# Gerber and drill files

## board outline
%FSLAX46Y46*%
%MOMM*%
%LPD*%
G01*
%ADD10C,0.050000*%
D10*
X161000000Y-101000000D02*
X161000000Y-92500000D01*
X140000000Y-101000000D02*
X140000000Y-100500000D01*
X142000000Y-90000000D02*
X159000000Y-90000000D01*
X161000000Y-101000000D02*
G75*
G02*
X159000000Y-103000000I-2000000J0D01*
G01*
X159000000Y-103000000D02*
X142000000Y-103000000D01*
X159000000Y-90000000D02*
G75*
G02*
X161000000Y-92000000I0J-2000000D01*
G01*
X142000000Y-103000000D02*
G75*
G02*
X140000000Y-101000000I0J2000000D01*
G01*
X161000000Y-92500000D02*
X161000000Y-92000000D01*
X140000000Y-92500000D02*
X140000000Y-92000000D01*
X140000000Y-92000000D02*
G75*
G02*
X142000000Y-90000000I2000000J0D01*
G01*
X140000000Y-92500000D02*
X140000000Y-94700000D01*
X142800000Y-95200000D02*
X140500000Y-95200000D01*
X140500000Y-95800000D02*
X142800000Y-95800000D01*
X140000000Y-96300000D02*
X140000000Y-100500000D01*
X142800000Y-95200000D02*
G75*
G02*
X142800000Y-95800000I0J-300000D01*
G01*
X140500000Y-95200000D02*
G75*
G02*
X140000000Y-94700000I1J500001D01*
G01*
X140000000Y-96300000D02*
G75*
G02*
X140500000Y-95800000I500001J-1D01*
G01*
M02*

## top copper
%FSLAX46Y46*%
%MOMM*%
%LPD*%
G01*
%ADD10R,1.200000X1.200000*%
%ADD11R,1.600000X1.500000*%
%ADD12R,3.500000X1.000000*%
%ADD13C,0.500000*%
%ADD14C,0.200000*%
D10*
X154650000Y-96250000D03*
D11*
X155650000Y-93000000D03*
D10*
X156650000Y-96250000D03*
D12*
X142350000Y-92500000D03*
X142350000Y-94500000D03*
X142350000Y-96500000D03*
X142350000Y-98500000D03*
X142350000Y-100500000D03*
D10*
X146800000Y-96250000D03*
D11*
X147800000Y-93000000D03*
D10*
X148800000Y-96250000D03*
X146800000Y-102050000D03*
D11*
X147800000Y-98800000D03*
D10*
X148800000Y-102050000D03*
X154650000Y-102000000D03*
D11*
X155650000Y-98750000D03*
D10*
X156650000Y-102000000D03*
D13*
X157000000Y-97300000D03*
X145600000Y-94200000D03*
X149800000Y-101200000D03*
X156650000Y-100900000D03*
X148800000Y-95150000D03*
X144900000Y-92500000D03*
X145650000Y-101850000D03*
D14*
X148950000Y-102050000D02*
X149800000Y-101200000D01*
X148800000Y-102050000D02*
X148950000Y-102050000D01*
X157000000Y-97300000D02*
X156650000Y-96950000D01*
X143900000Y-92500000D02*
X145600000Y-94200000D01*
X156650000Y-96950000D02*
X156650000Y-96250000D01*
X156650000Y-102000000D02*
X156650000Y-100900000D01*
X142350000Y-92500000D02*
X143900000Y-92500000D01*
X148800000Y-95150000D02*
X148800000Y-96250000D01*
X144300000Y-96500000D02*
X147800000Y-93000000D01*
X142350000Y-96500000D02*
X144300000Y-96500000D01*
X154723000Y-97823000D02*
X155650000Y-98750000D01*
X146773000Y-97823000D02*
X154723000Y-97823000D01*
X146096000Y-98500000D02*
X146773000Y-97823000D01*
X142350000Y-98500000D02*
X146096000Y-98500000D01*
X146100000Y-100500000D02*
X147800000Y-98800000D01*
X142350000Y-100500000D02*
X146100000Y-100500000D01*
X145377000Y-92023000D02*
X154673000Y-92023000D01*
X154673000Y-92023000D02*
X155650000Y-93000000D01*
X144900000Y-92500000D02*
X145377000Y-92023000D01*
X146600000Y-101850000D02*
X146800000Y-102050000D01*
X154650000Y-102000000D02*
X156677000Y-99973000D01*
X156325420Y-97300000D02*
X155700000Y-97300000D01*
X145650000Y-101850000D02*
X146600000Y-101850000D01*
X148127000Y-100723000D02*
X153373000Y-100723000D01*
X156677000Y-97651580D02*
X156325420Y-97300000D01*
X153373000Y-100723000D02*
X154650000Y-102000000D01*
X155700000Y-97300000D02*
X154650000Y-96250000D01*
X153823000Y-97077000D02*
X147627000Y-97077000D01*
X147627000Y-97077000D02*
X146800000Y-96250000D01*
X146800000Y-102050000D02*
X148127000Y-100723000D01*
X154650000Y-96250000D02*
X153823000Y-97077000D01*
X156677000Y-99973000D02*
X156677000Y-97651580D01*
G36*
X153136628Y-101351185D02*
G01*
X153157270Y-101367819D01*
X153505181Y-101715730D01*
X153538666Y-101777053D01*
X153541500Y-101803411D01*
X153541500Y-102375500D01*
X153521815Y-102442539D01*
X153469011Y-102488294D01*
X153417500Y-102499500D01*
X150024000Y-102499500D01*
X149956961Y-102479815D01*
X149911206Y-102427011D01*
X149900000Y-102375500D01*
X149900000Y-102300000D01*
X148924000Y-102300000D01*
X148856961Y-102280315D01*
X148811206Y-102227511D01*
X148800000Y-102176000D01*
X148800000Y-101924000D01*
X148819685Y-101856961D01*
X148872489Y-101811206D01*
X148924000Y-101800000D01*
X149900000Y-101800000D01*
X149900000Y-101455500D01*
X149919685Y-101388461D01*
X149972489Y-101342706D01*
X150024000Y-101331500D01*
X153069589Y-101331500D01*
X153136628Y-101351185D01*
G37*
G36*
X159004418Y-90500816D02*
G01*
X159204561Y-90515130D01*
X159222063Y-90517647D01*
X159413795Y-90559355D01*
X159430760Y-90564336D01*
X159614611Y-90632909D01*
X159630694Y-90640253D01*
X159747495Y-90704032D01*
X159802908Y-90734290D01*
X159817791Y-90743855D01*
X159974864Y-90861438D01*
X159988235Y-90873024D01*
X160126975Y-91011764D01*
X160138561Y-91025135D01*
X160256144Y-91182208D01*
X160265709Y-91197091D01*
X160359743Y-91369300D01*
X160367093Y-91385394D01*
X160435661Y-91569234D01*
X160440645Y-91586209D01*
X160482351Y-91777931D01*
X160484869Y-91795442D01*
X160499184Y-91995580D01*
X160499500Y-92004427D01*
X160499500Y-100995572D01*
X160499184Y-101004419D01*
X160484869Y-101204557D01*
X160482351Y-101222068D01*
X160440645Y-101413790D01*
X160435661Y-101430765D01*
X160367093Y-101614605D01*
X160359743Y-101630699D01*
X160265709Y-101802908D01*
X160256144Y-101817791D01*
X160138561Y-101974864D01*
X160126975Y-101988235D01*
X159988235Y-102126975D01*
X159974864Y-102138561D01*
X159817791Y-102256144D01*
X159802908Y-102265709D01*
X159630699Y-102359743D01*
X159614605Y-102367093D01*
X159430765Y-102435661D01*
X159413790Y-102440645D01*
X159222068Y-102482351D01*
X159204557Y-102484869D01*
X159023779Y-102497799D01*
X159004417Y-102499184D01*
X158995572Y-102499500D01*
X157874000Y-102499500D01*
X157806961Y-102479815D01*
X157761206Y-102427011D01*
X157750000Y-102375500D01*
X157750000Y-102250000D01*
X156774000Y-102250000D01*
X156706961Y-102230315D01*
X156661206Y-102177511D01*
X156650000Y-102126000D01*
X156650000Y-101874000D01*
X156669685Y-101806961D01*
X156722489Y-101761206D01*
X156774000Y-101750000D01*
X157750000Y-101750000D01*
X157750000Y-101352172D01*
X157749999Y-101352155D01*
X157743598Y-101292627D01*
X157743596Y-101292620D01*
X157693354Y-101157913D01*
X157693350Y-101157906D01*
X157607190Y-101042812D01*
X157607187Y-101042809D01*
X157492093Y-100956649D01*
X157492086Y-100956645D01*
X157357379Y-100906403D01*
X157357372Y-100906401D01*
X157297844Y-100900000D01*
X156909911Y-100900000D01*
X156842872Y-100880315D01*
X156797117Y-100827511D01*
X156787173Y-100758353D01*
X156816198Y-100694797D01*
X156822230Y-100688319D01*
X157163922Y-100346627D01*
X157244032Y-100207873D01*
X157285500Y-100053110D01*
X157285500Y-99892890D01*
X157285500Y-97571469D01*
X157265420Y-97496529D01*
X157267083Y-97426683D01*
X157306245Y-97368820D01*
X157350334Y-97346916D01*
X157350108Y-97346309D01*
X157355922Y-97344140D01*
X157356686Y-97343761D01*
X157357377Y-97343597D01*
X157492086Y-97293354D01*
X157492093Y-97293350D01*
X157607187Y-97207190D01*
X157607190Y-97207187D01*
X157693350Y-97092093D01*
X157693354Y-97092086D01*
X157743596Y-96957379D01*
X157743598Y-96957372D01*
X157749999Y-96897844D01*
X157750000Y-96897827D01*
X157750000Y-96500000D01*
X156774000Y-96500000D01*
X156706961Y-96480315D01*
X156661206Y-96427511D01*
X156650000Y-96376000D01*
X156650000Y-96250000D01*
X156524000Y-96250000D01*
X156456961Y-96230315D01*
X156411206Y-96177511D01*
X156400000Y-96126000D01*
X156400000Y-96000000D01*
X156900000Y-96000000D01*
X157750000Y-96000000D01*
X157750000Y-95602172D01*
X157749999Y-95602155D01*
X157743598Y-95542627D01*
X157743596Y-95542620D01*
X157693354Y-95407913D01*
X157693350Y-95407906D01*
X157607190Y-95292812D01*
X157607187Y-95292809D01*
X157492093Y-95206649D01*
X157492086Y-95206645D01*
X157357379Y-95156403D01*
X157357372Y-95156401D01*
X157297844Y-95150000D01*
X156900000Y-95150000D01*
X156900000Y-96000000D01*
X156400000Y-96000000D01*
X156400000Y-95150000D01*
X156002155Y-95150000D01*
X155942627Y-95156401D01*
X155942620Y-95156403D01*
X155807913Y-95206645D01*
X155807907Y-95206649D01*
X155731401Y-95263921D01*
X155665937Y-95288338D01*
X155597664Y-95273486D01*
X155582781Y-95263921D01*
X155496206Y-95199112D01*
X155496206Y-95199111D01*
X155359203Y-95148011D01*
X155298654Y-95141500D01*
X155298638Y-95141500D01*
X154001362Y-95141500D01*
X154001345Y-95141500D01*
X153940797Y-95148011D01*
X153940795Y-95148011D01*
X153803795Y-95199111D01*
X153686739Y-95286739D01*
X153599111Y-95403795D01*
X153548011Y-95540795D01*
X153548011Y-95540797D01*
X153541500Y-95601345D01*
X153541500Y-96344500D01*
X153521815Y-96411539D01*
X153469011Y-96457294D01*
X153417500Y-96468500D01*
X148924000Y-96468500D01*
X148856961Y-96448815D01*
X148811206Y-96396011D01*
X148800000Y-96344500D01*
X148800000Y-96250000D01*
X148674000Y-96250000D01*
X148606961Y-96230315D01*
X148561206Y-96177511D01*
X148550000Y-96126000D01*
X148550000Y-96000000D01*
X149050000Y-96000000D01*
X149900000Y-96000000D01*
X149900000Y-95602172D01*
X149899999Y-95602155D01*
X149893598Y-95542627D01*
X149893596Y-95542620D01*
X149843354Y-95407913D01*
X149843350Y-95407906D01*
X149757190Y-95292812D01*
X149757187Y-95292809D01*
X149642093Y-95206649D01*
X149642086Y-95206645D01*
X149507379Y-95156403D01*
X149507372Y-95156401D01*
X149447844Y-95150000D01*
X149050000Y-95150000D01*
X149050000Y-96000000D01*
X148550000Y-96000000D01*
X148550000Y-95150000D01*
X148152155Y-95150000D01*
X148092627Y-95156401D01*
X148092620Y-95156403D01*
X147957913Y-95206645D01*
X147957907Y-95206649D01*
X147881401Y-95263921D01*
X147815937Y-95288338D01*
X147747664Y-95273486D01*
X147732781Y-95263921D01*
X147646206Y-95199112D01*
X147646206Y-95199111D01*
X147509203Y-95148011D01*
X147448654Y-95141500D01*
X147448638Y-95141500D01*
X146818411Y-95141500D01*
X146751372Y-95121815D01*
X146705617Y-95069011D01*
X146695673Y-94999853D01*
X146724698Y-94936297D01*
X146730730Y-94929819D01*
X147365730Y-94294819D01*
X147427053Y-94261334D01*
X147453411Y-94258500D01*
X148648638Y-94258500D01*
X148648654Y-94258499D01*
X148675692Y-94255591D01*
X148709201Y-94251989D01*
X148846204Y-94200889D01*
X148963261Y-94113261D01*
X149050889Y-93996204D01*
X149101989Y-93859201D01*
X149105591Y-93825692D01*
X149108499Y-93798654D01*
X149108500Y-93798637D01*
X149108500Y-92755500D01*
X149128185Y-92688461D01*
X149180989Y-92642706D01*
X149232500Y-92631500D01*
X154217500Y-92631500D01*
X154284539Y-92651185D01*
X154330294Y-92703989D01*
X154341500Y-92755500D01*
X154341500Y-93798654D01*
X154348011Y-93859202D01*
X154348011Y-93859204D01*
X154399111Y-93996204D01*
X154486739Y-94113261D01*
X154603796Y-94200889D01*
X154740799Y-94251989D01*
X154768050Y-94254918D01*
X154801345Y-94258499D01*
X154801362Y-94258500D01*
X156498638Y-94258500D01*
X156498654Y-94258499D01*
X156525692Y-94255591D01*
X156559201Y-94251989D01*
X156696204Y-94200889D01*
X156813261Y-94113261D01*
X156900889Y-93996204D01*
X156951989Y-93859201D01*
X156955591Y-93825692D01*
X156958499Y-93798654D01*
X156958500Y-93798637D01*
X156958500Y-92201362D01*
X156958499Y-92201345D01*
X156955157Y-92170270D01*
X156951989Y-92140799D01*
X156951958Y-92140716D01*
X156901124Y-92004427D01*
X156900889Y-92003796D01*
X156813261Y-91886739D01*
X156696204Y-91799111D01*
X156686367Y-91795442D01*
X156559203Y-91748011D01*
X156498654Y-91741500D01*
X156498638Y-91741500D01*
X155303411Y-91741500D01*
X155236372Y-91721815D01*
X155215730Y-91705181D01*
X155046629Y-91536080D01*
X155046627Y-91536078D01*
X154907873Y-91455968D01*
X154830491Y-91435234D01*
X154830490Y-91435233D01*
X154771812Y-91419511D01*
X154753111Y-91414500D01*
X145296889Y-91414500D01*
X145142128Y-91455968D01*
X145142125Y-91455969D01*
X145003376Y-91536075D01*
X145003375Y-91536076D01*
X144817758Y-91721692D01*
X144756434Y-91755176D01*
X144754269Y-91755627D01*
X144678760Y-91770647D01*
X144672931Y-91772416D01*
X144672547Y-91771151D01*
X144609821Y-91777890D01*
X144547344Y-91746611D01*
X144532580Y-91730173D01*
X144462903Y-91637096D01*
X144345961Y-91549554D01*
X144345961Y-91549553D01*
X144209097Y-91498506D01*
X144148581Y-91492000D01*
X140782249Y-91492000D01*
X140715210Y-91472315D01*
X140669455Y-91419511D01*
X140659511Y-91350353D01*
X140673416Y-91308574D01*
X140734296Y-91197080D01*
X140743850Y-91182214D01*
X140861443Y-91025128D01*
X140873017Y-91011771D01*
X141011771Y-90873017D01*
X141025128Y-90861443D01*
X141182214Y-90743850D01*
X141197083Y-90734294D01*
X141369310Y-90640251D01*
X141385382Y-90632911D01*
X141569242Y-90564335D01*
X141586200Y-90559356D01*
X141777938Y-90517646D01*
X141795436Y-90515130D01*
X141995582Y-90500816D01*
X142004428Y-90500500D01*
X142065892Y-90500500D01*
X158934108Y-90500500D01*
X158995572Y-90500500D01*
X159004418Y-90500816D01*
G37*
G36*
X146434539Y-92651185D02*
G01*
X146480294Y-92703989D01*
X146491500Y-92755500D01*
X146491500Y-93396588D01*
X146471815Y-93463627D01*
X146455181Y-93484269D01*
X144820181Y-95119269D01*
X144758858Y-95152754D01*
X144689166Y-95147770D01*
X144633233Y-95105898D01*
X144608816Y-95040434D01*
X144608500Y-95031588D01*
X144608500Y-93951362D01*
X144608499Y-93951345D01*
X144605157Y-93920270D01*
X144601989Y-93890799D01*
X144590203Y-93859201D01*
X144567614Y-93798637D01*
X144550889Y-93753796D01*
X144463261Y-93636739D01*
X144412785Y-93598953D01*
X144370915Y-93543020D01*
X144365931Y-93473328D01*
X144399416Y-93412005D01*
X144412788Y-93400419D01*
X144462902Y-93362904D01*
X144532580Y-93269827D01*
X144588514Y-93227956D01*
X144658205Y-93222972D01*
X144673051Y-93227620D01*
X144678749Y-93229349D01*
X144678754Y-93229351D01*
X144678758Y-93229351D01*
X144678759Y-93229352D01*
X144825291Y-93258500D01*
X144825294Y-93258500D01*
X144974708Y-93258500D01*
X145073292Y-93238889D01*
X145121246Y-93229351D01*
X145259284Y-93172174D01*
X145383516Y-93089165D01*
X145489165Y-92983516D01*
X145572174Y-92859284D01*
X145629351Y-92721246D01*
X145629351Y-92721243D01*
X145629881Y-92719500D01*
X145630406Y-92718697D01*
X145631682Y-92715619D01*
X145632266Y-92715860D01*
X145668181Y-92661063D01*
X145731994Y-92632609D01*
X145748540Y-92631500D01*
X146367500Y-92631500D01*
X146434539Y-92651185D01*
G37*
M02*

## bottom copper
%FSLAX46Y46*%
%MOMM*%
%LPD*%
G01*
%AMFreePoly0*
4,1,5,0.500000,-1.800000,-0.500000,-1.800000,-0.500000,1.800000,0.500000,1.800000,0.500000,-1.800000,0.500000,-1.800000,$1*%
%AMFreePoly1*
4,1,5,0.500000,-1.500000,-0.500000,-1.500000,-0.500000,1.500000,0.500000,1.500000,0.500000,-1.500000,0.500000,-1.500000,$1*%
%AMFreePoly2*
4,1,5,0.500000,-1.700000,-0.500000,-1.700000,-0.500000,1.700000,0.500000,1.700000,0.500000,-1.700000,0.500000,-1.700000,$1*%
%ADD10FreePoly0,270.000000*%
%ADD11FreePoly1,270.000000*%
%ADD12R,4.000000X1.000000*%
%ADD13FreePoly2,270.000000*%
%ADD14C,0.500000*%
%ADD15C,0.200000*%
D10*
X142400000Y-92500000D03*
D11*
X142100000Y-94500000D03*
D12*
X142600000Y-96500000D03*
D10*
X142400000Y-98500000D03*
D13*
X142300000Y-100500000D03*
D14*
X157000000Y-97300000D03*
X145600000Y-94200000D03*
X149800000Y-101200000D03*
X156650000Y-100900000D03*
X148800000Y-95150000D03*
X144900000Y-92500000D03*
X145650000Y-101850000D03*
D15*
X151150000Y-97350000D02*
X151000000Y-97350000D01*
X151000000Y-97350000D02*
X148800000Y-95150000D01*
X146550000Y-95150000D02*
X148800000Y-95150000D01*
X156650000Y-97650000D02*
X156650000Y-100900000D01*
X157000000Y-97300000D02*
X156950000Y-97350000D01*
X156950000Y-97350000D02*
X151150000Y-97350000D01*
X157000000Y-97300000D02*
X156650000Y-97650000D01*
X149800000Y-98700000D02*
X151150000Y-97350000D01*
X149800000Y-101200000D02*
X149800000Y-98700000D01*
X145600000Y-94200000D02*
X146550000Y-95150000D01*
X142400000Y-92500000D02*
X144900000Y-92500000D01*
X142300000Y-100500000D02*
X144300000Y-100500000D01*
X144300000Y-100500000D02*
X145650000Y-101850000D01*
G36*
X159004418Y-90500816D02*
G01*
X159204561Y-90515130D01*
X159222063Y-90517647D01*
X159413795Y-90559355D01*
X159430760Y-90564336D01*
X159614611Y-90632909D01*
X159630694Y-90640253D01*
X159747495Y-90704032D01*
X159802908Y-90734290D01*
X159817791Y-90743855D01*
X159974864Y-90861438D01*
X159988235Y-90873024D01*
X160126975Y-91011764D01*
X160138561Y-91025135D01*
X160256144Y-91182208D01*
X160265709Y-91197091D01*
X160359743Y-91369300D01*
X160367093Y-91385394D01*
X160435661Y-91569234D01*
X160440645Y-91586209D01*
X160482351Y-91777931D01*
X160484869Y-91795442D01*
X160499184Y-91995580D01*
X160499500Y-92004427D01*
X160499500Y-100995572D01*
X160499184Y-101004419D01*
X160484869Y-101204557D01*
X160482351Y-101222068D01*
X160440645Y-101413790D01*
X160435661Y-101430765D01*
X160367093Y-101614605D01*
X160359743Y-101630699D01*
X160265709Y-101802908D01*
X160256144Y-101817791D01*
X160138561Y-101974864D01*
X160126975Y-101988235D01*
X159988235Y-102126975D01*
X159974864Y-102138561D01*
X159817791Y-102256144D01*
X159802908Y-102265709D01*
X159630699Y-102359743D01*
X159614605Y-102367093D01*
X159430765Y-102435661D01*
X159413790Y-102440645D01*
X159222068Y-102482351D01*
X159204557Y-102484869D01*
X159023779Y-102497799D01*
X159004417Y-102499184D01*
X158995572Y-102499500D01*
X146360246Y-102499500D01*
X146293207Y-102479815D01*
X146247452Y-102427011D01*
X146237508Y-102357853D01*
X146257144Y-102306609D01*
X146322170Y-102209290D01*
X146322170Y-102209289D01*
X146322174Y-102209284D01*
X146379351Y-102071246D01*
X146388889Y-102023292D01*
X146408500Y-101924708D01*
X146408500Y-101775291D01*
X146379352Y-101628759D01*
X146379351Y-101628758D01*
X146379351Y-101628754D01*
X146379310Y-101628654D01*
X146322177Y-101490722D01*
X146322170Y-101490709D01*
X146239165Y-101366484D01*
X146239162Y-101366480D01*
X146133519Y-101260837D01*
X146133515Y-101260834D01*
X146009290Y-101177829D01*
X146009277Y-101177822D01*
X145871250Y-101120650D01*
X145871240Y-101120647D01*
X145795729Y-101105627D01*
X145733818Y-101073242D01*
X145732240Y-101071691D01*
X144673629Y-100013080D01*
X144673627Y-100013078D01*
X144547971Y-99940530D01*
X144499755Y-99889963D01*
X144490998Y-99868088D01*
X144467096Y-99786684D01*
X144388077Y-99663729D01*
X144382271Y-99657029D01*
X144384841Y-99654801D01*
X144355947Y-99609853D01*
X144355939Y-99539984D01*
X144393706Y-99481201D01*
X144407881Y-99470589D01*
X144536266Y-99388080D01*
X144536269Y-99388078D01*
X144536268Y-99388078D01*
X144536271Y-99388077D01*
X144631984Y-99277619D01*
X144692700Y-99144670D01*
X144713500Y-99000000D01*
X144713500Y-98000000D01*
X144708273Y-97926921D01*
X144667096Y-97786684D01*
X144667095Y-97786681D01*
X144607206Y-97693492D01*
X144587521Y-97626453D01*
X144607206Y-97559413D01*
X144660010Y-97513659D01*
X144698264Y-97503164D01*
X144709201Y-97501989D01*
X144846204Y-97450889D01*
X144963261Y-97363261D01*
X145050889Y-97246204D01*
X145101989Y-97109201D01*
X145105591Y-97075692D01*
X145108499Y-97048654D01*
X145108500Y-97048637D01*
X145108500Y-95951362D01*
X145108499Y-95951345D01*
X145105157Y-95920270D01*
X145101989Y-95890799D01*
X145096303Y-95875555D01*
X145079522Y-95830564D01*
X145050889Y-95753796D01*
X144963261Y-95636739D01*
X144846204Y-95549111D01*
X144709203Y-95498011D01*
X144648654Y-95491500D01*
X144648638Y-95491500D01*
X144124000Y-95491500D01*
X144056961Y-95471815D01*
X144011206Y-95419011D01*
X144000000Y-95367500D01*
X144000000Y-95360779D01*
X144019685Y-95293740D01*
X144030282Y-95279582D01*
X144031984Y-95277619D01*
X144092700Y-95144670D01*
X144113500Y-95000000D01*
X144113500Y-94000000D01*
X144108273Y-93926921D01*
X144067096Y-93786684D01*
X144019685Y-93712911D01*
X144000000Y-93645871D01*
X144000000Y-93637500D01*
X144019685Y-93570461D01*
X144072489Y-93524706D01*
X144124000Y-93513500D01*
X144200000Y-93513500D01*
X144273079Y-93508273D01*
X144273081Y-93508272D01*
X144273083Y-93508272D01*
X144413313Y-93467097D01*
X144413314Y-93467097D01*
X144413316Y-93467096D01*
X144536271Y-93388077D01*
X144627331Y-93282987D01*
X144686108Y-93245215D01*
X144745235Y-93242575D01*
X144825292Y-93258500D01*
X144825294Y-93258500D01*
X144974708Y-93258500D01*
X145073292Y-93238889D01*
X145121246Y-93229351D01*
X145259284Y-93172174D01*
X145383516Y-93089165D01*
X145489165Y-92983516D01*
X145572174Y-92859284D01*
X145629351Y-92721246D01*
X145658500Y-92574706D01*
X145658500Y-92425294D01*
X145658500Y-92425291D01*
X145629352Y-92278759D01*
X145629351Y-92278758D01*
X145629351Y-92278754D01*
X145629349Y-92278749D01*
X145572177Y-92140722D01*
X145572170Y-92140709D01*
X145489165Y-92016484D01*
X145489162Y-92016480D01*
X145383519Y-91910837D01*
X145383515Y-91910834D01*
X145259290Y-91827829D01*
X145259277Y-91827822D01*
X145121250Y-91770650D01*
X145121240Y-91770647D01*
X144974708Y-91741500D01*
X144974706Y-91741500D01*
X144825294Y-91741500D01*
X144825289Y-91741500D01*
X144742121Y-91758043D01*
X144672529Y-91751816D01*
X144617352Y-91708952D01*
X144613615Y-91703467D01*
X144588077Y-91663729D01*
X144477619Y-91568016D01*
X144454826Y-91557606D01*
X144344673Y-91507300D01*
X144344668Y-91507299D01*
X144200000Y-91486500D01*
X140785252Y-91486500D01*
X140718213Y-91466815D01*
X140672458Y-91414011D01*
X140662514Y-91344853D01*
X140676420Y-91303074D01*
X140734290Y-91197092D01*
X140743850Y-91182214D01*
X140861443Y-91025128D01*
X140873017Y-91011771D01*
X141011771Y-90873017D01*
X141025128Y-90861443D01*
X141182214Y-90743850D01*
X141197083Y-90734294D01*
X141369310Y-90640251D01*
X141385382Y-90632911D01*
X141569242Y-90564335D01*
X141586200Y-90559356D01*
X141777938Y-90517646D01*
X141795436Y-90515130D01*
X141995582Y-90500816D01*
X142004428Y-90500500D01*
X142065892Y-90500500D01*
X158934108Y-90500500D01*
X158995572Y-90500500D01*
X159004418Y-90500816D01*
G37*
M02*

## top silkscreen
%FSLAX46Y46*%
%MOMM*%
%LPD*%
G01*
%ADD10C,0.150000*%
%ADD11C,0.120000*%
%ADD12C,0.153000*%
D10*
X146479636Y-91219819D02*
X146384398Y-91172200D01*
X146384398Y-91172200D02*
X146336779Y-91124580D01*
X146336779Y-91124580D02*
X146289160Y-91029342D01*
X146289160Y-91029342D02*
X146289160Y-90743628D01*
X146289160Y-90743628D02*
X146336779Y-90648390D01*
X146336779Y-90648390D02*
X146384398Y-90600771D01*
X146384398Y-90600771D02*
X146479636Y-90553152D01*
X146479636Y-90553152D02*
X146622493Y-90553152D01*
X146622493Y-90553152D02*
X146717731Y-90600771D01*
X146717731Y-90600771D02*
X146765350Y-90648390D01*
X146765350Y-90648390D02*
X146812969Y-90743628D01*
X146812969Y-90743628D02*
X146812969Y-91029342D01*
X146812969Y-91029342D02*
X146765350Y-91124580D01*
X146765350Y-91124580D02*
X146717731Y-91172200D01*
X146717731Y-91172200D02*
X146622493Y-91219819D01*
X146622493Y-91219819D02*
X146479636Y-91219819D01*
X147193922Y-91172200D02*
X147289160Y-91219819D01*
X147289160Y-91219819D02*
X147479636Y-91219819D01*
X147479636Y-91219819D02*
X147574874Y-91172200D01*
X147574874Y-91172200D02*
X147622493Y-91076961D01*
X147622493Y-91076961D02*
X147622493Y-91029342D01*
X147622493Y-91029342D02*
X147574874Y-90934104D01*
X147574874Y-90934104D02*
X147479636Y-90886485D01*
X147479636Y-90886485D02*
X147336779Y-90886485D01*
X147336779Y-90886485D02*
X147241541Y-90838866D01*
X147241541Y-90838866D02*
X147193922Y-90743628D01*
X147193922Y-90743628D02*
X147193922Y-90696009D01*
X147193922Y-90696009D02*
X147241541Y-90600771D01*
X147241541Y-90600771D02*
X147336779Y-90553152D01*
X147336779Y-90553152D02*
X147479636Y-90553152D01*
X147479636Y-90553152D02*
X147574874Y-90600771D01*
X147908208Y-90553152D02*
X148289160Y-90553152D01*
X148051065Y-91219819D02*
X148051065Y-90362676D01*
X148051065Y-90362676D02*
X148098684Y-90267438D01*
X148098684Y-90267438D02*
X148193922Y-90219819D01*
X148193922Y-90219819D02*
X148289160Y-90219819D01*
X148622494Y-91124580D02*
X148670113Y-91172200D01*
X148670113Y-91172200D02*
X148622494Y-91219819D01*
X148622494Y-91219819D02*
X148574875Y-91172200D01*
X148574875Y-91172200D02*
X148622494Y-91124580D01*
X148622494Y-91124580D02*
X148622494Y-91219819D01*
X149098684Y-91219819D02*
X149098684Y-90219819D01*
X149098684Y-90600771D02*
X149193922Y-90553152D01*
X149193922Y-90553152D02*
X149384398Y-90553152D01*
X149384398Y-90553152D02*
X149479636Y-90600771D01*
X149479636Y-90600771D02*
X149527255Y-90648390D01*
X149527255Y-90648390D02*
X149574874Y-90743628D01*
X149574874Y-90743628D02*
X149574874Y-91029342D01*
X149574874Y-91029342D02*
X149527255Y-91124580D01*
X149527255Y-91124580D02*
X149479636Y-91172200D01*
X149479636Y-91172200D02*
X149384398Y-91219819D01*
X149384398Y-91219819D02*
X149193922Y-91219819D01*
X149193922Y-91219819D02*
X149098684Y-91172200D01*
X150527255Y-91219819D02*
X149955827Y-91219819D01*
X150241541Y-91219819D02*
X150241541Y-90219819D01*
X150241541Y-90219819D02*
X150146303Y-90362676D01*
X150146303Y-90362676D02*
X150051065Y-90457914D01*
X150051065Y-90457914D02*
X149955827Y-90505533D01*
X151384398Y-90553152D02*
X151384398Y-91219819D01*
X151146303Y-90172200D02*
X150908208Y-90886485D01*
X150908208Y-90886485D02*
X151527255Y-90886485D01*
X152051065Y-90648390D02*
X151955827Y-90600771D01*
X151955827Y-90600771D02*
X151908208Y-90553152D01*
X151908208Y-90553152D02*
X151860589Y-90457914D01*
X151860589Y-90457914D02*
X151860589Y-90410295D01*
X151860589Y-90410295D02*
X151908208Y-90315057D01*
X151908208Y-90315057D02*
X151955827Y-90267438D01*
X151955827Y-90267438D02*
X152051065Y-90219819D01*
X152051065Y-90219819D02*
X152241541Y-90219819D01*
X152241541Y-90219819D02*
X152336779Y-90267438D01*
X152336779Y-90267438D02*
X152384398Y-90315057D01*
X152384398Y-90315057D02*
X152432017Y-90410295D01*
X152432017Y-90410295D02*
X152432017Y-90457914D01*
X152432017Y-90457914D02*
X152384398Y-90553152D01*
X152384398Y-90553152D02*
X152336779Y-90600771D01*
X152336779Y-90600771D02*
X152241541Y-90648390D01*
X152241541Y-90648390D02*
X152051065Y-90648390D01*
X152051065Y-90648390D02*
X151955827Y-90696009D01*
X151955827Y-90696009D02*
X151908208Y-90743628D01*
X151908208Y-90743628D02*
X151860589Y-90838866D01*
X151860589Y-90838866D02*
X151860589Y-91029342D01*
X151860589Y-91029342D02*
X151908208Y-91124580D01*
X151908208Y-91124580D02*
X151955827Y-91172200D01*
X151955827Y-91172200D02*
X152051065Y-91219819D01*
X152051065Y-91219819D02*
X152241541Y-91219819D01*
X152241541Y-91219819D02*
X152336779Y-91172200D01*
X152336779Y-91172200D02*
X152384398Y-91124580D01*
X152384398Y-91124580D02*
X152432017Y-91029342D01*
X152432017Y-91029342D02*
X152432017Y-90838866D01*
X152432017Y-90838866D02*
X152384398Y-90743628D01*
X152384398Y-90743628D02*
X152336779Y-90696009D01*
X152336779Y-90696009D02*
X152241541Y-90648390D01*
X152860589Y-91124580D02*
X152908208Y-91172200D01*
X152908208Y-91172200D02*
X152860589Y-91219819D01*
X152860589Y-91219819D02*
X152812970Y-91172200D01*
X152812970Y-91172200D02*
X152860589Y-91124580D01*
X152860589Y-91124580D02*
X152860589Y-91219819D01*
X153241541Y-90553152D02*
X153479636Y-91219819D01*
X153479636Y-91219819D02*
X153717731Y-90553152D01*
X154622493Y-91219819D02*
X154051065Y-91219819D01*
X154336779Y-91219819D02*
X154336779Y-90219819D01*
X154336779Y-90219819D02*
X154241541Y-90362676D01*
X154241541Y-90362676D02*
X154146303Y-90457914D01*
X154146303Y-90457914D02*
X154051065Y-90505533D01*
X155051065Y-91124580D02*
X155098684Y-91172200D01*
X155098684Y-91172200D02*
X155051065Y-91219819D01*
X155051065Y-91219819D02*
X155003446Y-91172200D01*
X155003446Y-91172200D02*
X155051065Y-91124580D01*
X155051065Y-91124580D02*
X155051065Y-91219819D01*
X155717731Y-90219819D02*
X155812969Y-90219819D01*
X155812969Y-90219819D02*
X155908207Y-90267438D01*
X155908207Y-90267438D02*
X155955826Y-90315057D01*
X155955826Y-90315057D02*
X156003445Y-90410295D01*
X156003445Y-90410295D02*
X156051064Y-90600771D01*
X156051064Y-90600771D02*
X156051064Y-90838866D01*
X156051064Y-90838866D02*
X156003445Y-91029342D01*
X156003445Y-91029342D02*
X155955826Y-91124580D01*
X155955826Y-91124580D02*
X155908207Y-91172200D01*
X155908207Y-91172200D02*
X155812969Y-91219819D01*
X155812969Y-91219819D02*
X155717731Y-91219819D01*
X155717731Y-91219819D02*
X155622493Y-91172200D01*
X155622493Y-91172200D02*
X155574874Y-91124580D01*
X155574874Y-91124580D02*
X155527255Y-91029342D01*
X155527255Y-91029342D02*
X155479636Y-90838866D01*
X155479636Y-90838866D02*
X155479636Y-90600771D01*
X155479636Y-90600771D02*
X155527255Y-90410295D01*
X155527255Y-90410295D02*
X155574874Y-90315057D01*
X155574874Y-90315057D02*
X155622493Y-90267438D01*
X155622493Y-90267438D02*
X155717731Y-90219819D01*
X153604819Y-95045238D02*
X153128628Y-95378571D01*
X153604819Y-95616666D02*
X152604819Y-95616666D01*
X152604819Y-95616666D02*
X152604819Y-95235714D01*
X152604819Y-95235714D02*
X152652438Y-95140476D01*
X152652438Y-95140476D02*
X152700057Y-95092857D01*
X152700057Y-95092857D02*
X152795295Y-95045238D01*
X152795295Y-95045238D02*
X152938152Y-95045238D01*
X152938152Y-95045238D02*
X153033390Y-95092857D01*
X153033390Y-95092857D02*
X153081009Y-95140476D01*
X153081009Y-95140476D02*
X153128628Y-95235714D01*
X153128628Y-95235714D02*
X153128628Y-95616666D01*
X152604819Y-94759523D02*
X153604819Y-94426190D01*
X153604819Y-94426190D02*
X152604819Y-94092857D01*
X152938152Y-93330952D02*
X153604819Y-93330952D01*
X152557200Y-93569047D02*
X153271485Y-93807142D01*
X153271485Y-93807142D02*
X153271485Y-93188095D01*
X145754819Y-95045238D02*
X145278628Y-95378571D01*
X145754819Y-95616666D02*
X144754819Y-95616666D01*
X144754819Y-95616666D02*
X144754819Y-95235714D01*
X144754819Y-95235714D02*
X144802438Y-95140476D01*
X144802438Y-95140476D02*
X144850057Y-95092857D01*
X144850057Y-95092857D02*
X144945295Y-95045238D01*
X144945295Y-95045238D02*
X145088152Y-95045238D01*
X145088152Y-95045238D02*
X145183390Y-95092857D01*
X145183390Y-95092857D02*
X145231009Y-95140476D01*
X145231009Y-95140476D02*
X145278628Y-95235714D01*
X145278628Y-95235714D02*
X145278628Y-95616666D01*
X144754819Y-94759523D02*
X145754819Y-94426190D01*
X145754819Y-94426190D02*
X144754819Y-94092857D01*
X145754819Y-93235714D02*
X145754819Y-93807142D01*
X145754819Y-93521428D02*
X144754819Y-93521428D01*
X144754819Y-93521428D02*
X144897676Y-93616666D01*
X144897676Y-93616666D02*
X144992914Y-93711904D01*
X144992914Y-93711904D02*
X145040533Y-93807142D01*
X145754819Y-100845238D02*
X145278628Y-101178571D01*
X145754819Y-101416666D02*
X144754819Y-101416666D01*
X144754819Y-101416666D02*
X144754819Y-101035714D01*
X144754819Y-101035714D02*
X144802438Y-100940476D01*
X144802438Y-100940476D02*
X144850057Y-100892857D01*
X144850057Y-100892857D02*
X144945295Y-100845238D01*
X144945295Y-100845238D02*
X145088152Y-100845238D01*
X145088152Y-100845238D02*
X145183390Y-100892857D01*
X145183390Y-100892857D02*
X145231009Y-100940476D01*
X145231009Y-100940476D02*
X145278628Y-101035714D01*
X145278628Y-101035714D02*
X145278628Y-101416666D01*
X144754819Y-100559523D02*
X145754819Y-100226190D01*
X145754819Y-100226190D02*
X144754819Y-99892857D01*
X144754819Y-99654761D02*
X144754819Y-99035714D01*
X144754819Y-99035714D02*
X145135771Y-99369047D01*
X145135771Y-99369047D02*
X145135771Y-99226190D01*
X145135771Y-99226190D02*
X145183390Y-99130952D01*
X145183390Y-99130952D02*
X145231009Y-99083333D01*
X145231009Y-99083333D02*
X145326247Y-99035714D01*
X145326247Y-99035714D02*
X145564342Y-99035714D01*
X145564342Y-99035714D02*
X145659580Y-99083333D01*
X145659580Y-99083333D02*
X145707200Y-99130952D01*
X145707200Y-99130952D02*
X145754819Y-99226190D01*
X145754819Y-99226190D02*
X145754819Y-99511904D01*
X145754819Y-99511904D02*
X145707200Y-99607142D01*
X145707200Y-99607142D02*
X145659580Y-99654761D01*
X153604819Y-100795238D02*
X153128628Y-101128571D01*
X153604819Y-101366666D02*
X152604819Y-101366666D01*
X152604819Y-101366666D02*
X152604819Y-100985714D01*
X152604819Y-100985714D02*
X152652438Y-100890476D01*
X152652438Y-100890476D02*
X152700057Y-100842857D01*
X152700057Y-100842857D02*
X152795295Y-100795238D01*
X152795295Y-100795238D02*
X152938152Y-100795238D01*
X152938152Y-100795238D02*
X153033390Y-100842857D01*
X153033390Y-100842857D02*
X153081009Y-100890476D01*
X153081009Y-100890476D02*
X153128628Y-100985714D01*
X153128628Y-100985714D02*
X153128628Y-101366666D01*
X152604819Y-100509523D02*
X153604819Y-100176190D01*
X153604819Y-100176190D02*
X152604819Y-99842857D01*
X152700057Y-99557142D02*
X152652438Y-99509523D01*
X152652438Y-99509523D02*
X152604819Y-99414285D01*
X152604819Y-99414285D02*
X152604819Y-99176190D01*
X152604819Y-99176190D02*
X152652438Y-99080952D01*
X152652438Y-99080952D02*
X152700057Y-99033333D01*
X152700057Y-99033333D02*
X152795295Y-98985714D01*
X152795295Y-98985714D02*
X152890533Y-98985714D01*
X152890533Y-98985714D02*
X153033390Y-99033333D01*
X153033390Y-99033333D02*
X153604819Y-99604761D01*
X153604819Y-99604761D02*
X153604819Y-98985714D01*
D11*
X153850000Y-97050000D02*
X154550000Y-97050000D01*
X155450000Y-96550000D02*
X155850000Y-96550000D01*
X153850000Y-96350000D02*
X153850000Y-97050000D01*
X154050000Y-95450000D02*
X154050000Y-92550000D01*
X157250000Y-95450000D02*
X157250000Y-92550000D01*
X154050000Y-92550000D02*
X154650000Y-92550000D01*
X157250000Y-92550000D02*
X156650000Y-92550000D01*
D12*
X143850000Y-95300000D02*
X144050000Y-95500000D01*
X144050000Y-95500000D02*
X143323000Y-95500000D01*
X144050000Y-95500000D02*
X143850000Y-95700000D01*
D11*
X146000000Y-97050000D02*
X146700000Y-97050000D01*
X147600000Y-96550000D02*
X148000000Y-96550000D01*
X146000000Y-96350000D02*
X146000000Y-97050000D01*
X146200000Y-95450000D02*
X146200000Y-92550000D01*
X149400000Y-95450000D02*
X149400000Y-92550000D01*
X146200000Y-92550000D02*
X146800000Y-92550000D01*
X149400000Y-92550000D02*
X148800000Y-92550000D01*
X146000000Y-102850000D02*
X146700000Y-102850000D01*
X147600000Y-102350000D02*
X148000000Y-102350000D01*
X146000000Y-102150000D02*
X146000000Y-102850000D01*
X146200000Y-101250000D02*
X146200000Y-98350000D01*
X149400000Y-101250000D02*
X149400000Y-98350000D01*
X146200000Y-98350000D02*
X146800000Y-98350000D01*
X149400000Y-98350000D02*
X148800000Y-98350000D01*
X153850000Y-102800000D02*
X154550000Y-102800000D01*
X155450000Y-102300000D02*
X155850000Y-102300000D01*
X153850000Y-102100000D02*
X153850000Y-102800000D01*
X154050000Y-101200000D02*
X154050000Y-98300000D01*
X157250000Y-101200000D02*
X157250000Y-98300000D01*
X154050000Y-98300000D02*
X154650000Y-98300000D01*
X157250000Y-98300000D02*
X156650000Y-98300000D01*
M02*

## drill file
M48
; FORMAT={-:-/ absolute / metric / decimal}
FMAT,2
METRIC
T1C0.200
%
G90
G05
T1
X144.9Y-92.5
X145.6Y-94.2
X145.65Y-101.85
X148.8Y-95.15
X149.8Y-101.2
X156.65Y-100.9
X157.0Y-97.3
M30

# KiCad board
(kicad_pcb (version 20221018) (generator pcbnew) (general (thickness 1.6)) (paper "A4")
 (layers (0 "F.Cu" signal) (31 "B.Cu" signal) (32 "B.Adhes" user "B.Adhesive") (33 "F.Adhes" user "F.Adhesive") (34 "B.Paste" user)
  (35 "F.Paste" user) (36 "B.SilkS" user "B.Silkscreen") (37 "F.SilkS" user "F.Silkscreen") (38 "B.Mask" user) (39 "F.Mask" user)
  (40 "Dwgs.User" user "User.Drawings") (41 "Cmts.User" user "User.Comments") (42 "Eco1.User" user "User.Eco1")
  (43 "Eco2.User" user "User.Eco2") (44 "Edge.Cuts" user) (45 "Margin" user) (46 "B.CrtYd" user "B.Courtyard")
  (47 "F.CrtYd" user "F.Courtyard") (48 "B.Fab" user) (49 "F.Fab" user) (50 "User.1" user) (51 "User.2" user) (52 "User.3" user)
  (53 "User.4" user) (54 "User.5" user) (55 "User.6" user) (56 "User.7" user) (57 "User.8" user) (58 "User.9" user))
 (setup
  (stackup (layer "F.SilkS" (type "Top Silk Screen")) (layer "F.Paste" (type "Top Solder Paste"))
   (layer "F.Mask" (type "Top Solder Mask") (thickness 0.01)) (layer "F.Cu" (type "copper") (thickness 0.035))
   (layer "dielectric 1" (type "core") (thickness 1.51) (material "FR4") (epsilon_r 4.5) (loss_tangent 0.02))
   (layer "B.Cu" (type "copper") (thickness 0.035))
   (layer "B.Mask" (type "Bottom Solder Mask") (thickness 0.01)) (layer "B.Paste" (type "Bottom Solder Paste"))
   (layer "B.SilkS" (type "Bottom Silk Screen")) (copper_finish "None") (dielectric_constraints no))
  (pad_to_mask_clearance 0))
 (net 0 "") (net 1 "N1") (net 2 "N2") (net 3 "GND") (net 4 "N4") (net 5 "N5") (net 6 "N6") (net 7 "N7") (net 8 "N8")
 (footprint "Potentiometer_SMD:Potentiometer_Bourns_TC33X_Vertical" (layer "F.Cu") (at 155.65 94.45 90)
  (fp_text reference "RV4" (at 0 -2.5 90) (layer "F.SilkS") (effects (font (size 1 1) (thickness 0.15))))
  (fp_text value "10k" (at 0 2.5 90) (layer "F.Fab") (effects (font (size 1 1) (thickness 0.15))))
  (fp_line (start -2.6 -1.8) (end -2.6 -1.1) (stroke (width 0.12) (type solid)) (layer "F.SilkS"))
  (fp_line (start -2.1 -0.2) (end -2.1 0.2) (stroke (width 0.12) (type solid)) (layer "F.SilkS"))
  (fp_line (start -1.9 -1.8) (end -2.6 -1.8) (stroke (width 0.12) (type solid)) (layer "F.SilkS"))
  (fp_line (start -1 -1.6) (end 1.9 -1.6) (stroke (width 0.12) (type solid)) (layer "F.SilkS"))
  (fp_line (start -1 1.6) (end 1.9 1.6) (stroke (width 0.12) (type solid)) (layer "F.SilkS"))
  (fp_line (start 1.9 -1.6) (end 1.9 -1) (stroke (width 0.12) (type solid)) (layer "F.SilkS"))
  (fp_line (start 1.9 1.6) (end 1.9 1) (stroke (width 0.12) (type solid)) (layer "F.SilkS"))
  (pad "1" smd rect (at -1.8 -1 90) (size 1.2 1.2) (layers "F.Cu" "F.Paste" "F.Mask") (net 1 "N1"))
  (pad "2" smd rect (at 1.45 0 90) (size 1.5 1.6) (layers "F.Cu" "F.Paste" "F.Mask") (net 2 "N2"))
  (pad "3" smd rect (at -1.8 1 90) (size 1.2 1.2) (layers "F.Cu" "F.Paste" "F.Mask") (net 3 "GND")))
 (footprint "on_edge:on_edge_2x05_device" (layer "F.Cu") (at 140 96.5 -90)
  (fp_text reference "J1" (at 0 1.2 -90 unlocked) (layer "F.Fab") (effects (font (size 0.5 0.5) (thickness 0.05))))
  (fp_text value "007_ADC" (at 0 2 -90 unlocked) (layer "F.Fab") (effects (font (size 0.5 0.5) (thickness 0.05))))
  (fp_line (start -1.2 -3.85) (end -1 -4.05) (stroke (width 0.153) (type solid)) (layer "F.SilkS"))
  (fp_line (start -1 -4.05) (end -1 -3.323) (stroke (width 0.153) (type solid)) (layer "F.SilkS"))
  (fp_line (start -1 -4.05) (end -0.8 -3.85) (stroke (width 0.153) (type solid)) (layer "F.SilkS"))
  (fp_line (start -4 0) (end -1.8 0) (stroke (width 0.05) (type solid)) (layer "Edge.Cuts"))
  (fp_line (start -1.3 -2.8) (end -1.3 -0.5) (stroke (width 0.05) (type solid)) (layer "Edge.Cuts"))
  (fp_line (start -0.7 -0.5) (end -0.7 -2.8) (stroke (width 0.05) (type solid)) (layer "Edge.Cuts"))
  (fp_line (start -0.2 0) (end 4 0) (stroke (width 0.05) (type solid)) (layer "Edge.Cuts"))
  (fp_arc (start -1.3 -2.8) (mid -1 -3.1) (end -0.7 -2.8) (stroke (width 0.05) (type solid)) (layer "Edge.Cuts"))
  (fp_arc (start -1.3 -0.5) (mid -1.446447 -0.146447) (end -1.8 0) (stroke (width 0.05) (type solid)) (layer "Edge.Cuts"))
  (fp_arc (start -0.2 0) (mid -0.553553 -0.146447) (end -0.7 -0.5) (stroke (width 0.05) (type solid)) (layer "Edge.Cuts"))
  (pad "1" smd rect (at -4 -2.35 90) (size 1 3.5) (layers "F.Cu" "F.Mask") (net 3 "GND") (zone_connect 0))
  (pad "2" smd rect (at -2 -2.35 270) (size 1 3.5) (layers "F.Cu" "F.Mask") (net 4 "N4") (zone_connect 0))
  (pad "3" smd rect (at 0 -2.35 270) (size 1 3.5) (layers "F.Cu" "F.Mask") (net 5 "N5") (zone_connect 0))
  (pad "4" smd rect (at 2 -2.35 90) (size 1 3.5) (layers "F.Cu" "F.Mask") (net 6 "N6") (zone_connect 0))
  (pad "5" smd rect (at 4 -2.35 90) (size 1 3.5) (layers "F.Cu" "F.Mask") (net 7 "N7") (zone_connect 0))
  (pad "6" smd custom (at -4 -2.4 270) (size 1 3.6) (layers "B.Cu" "B.Mask") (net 2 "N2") (zone_connect 0)
   (options (clearance outline) (anchor rect)) (primitives))
  (pad "7" smd custom (at -2 -2.1 270) (size 1 3) (layers "B.Cu" "B.Mask") (zone_connect 0) (options (clearance outline) (anchor rect))
   (primitives))
  (pad "8" smd rect (at 0 -2.6 270) (size 1 4) (layers "B.Cu" "B.Mask") (zone_connect 0))
  (pad "9" smd custom (at 2 -2.4 270) (size 1 3.6) (layers "B.Cu" "B.Mask") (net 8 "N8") (zone_connect 0)
   (options (clearance outline) (anchor rect)) (primitives))
  (pad "10" smd custom (at 4 -2.3 270) (size 1 3.4) (layers "B.Cu" "B.Mask") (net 1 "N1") (zone_connect 0)
   (options (clearance outline) (anchor rect)) (primitives))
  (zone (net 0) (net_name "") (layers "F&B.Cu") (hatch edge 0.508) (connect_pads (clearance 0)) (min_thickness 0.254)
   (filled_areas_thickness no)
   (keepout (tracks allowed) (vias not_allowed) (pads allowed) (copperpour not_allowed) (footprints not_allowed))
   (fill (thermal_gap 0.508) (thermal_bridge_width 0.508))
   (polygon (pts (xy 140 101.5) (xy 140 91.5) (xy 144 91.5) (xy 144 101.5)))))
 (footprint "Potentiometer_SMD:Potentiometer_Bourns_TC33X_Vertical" (layer "F.Cu") (at 147.8 94.45 90)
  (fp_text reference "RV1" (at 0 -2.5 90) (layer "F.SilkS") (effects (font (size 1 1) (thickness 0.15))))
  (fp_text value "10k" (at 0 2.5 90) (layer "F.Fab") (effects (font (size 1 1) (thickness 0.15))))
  (fp_line (start -2.6 -1.8) (end -2.6 -1.1) (stroke (width 0.12) (type solid)) (layer "F.SilkS"))
  (fp_line (start -2.1 -0.2) (end -2.1 0.2) (stroke (width 0.12) (type solid)) (layer "F.SilkS"))
  (fp_line (start -1.9 -1.8) (end -2.6 -1.8) (stroke (width 0.12) (type solid)) (layer "F.SilkS"))
  (fp_line (start -1 -1.6) (end 1.9 -1.6) (stroke (width 0.12) (type solid)) (layer "F.SilkS"))
  (fp_line (start -1 1.6) (end 1.9 1.6) (stroke (width 0.12) (type solid)) (layer "F.SilkS"))
  (fp_line (start 1.9 -1.6) (end 1.9 -1) (stroke (width 0.12) (type solid)) (layer "F.SilkS"))
  (fp_line (start 1.9 1.6) (end 1.9 1) (stroke (width 0.12) (type solid)) (layer "F.SilkS"))
  (pad "1" smd rect (at -1.8 -1 90) (size 1.2 1.2) (layers "F.Cu" "F.Paste" "F.Mask") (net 1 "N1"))
  (pad "2" smd rect (at 1.45 0 90) (size 1.5 1.6) (layers "F.Cu" "F.Paste" "F.Mask") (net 5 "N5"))
  (pad "3" smd rect (at -1.8 1 90) (size 1.2 1.2) (layers "F.Cu" "F.Paste" "F.Mask") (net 3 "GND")))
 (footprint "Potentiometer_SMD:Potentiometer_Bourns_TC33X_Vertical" (layer "F.Cu") (at 147.8 100.25 90)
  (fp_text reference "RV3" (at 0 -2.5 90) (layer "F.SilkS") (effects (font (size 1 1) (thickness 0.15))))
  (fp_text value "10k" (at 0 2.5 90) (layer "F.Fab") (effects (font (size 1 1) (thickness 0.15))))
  (fp_line (start -2.6 -1.8) (end -2.6 -1.1) (stroke (width 0.12) (type solid)) (layer "F.SilkS"))
  (fp_line (start -2.1 -0.2) (end -2.1 0.2) (stroke (width 0.12) (type solid)) (layer "F.SilkS"))
  (fp_line (start -1.9 -1.8) (end -2.6 -1.8) (stroke (width 0.12) (type solid)) (layer "F.SilkS"))
  (fp_line (start -1 -1.6) (end 1.9 -1.6) (stroke (width 0.12) (type solid)) (layer "F.SilkS"))
  (fp_line (start -1 1.6) (end 1.9 1.6) (stroke (width 0.12) (type solid)) (layer "F.SilkS"))
  (fp_line (start 1.9 -1.6) (end 1.9 -1) (stroke (width 0.12) (type solid)) (layer "F.SilkS"))
  (fp_line (start 1.9 1.6) (end 1.9 1) (stroke (width 0.12) (type solid)) (layer "F.SilkS"))
  (pad "1" smd rect (at -1.8 -1 90) (size 1.2 1.2) (layers "F.Cu" "F.Paste" "F.Mask") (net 1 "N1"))
  (pad "2" smd rect (at 1.45 0 90) (size 1.5 1.6) (layers "F.Cu" "F.Paste" "F.Mask") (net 7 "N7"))
  (pad "3" smd rect (at -1.8 1 90) (size 1.2 1.2) (layers "F.Cu" "F.Paste" "F.Mask") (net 3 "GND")))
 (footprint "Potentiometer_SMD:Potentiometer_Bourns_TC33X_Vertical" (layer "F.Cu") (at 155.65 100.2 90)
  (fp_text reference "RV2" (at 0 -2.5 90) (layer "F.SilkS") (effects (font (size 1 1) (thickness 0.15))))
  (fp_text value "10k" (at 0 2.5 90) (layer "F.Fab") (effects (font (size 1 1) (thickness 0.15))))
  (fp_line (start -2.6 -1.8) (end -2.6 -1.1) (stroke (width 0.12) (type solid)) (layer "F.SilkS"))
  (fp_line (start -2.1 -0.2) (end -2.1 0.2) (stroke (width 0.12) (type solid)) (layer "F.SilkS"))
  (fp_line (start -1.9 -1.8) (end -2.6 -1.8) (stroke (width 0.12) (type solid)) (layer "F.SilkS"))
  (fp_line (start -1 -1.6) (end 1.9 -1.6) (stroke (width 0.12) (type solid)) (layer "F.SilkS"))
  (fp_line (start -1 1.6) (end 1.9 1.6) (stroke (width 0.12) (type solid)) (layer "F.SilkS"))
  (fp_line (start 1.9 -1.6) (end 1.9 -1) (stroke (width 0.12) (type solid)) (layer "F.SilkS"))
  (fp_line (start 1.9 1.6) (end 1.9 1) (stroke (width 0.12) (type solid)) (layer "F.SilkS"))
  (pad "1" smd rect (at -1.8 -1 90) (size 1.2 1.2) (layers "F.Cu" "F.Paste" "F.Mask") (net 1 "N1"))
  (pad "2" smd rect (at 1.45 0 90) (size 1.5 1.6) (layers "F.Cu" "F.Paste" "F.Mask") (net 6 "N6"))
  (pad "3" smd rect (at -1.8 1 90) (size 1.2 1.2) (layers "F.Cu" "F.Paste" "F.Mask") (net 3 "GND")))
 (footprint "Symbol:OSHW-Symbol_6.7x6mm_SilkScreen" (layer "B.Cu") (at 151.75 99.35 180)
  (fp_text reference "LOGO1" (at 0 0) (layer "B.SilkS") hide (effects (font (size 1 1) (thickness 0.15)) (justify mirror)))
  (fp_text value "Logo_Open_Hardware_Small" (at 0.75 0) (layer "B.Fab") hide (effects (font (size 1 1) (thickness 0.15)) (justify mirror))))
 (gr_line (start 161 101) (end 161 92.5) (stroke (width 0.05) (type solid)) (layer "Edge.Cuts"))
 (gr_line (start 140 101) (end 140 100.5) (stroke (width 0.05) (type solid)) (layer "Edge.Cuts"))
 (gr_line (start 142 90) (end 159 90) (stroke (width 0.05) (type solid)) (layer "Edge.Cuts"))
 (gr_arc (start 161 101) (mid 160.414214 102.414214) (end 159 103) (stroke (width 0.05) (type solid)) (layer "Edge.Cuts"))
 (gr_line (start 159 103) (end 142 103) (stroke (width 0.05) (type solid)) (layer "Edge.Cuts"))
 (gr_arc (start 159 90) (mid 160.414214 90.585786) (end 161 92) (stroke (width 0.05) (type solid)) (layer "Edge.Cuts"))
 (gr_arc (start 142 103) (mid 140.585786 102.414214) (end 140 101) (stroke (width 0.05) (type solid)) (layer "Edge.Cuts"))
 (gr_line (start 161 92.5) (end 161 92) (stroke (width 0.05) (type solid)) (layer "Edge.Cuts"))
 (gr_line (start 140 92.5) (end 140 92) (stroke (width 0.05) (type solid)) (layer "Edge.Cuts"))
 (gr_arc (start 140 92) (mid 140.585786 90.585786) (end 142 90) (stroke (width 0.05) (type solid)) (layer "Edge.Cuts"))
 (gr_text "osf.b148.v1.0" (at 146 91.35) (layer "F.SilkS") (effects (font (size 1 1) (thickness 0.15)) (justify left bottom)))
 (segment (start 148.95 102.05) (end 149.8 101.2) (width 0.2) (layer "F.Cu") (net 3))
 (segment (start 148.8 102.05) (end 148.95 102.05) (width 0.2) (layer "F.Cu") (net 3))
 (segment (start 157 97.3) (end 156.65 96.95) (width 0.2) (layer "F.Cu") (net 3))
 (segment (start 143.9 92.5) (end 145.6 94.2) (width 0.2) (layer "F.Cu") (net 3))
 (segment (start 156.65 96.95) (end 156.65 96.25) (width 0.2) (layer "F.Cu") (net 3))
 (segment (start 156.65 102) (end 156.65 100.9) (width 0.2) (layer "F.Cu") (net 3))
 (segment (start 142.35 92.5) (end 143.9 92.5) (width 0.2) (layer "F.Cu") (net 3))
 (segment (start 148.8 95.15) (end 148.8 96.25) (width 0.2) (layer "F.Cu") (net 3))
 (via (at 157 97.3) (size 0.5) (drill 0.2) (layers "F.Cu" "B.Cu") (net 3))
 (via (at 145.6 94.2) (size 0.5) (drill 0.2) (layers "F.Cu" "B.Cu") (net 3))
 (via (at 149.8 101.2) (size 0.5) (drill 0.2) (layers "F.Cu" "B.Cu") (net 3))
 (via (at 156.65 100.9) (size 0.5) (drill 0.2) (layers "F.Cu" "B.Cu") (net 3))
 (via (at 148.8 95.15) (size 0.5) (drill 0.2) (layers "F.Cu" "B.Cu") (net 3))
 (segment (start 151.15 97.35) (end 151 97.35) (width 0.2) (layer "B.Cu") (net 3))
 (segment (start 151 97.35) (end 148.8 95.15) (width 0.2) (layer "B.Cu") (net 3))
 (segment (start 146.55 95.15) (end 148.8 95.15) (width 0.2) (layer "B.Cu") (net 3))
 (segment (start 156.65 97.65) (end 156.65 100.9) (width 0.2) (layer "B.Cu") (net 3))
 (segment (start 157 97.3) (end 156.95 97.35) (width 0.2) (layer "B.Cu") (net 3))
 (segment (start 156.95 97.35) (end 151.15 97.35) (width 0.2) (layer "B.Cu") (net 3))
 (segment (start 157 97.3) (end 156.65 97.65) (width 0.2) (layer "B.Cu") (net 3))
 (segment (start 149.8 98.7) (end 151.15 97.35) (width 0.2) (layer "B.Cu") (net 3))
 (segment (start 149.8 101.2) (end 149.8 98.7) (width 0.2) (layer "B.Cu") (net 3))
 (segment (start 145.6 94.2) (end 146.55 95.15) (width 0.2) (layer "B.Cu") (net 3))
 (segment (start 144.3 96.5) (end 147.8 93) (width 0.2) (layer "F.Cu") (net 5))
 (segment (start 142.35 96.5) (end 144.3 96.5) (width 0.2) (layer "F.Cu") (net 5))
 (segment (start 154.723 97.823) (end 155.65 98.75) (width 0.2) (layer "F.Cu") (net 6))
 (segment (start 146.773 97.823) (end 154.723 97.823) (width 0.2) (layer "F.Cu") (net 6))
 (segment (start 146.096 98.5) (end 146.773 97.823) (width 0.2) (layer "F.Cu") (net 6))
 (segment (start 142.35 98.5) (end 146.096 98.5) (width 0.2) (layer "F.Cu") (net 6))
 (segment (start 146.1 100.5) (end 147.8 98.8) (width 0.2) (layer "F.Cu") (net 7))
 (segment (start 142.35 100.5) (end 146.1 100.5) (width 0.2) (layer "F.Cu") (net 7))
 (segment (start 145.377 92.023) (end 154.673 92.023) (width 0.2) (layer "F.Cu") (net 2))
 (segment (start 154.673 92.023) (end 155.65 93) (width 0.2) (layer "F.Cu") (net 2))
 (segment (start 144.9 92.5) (end 145.377 92.023) (width 0.2) (layer "F.Cu") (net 2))
 (via (at 144.9 92.5) (size 0.5) (drill 0.2) (layers "F.Cu" "B.Cu") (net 2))
 (segment (start 142.4 92.5) (end 144.9 92.5) (width 0.2) (layer "B.Cu") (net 2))
 (segment (start 146.6 101.85) (end 146.8 102.05) (width 0.2) (layer "F.Cu") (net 1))
 (segment (start 154.65 102) (end 156.677 99.973) (width 0.2) (layer "F.Cu") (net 1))
 (segment (start 156.32542 97.3) (end 155.7 97.3) (width 0.2) (layer "F.Cu") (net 1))
 (segment (start 145.65 101.85) (end 146.6 101.85) (width 0.2) (layer "F.Cu") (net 1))
 (segment (start 148.127 100.723) (end 153.373 100.723) (width 0.2) (layer "F.Cu") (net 1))
 (segment (start 156.677 97.65158) (end 156.32542 97.3) (width 0.2) (layer "F.Cu") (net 1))
 (segment (start 153.373 100.723) (end 154.65 102) (width 0.2) (layer "F.Cu") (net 1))
 (segment (start 155.7 97.3) (end 154.65 96.25) (width 0.2) (layer "F.Cu") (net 1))
 (segment (start 153.823 97.077) (end 147.627 97.077) (width 0.2) (layer "F.Cu") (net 1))
 (segment (start 147.627 97.077) (end 146.8 96.25) (width 0.2) (layer "F.Cu") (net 1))
 (segment (start 146.8 102.05) (end 148.127 100.723) (width 0.2) (layer "F.Cu") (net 1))
 (segment (start 154.65 96.25) (end 153.823 97.077) (width 0.2) (layer "F.Cu") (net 1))
 (segment (start 156.677 99.973) (end 156.677 97.65158) (width 0.2) (layer "F.Cu") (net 1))
 (via (at 145.65 101.85) (size 0.5) (drill 0.2) (layers "F.Cu" "B.Cu") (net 1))
 (segment (start 142.3 100.5) (end 144.3 100.5) (width 0.2) (layer "B.Cu") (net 1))
 (segment (start 144.3 100.5) (end 145.65 101.85) (width 0.2) (layer "B.Cu") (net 1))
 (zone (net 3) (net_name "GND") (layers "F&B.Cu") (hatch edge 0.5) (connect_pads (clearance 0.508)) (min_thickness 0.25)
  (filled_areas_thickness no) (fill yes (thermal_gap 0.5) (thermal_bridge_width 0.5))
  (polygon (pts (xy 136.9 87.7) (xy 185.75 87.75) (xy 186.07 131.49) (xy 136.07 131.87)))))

